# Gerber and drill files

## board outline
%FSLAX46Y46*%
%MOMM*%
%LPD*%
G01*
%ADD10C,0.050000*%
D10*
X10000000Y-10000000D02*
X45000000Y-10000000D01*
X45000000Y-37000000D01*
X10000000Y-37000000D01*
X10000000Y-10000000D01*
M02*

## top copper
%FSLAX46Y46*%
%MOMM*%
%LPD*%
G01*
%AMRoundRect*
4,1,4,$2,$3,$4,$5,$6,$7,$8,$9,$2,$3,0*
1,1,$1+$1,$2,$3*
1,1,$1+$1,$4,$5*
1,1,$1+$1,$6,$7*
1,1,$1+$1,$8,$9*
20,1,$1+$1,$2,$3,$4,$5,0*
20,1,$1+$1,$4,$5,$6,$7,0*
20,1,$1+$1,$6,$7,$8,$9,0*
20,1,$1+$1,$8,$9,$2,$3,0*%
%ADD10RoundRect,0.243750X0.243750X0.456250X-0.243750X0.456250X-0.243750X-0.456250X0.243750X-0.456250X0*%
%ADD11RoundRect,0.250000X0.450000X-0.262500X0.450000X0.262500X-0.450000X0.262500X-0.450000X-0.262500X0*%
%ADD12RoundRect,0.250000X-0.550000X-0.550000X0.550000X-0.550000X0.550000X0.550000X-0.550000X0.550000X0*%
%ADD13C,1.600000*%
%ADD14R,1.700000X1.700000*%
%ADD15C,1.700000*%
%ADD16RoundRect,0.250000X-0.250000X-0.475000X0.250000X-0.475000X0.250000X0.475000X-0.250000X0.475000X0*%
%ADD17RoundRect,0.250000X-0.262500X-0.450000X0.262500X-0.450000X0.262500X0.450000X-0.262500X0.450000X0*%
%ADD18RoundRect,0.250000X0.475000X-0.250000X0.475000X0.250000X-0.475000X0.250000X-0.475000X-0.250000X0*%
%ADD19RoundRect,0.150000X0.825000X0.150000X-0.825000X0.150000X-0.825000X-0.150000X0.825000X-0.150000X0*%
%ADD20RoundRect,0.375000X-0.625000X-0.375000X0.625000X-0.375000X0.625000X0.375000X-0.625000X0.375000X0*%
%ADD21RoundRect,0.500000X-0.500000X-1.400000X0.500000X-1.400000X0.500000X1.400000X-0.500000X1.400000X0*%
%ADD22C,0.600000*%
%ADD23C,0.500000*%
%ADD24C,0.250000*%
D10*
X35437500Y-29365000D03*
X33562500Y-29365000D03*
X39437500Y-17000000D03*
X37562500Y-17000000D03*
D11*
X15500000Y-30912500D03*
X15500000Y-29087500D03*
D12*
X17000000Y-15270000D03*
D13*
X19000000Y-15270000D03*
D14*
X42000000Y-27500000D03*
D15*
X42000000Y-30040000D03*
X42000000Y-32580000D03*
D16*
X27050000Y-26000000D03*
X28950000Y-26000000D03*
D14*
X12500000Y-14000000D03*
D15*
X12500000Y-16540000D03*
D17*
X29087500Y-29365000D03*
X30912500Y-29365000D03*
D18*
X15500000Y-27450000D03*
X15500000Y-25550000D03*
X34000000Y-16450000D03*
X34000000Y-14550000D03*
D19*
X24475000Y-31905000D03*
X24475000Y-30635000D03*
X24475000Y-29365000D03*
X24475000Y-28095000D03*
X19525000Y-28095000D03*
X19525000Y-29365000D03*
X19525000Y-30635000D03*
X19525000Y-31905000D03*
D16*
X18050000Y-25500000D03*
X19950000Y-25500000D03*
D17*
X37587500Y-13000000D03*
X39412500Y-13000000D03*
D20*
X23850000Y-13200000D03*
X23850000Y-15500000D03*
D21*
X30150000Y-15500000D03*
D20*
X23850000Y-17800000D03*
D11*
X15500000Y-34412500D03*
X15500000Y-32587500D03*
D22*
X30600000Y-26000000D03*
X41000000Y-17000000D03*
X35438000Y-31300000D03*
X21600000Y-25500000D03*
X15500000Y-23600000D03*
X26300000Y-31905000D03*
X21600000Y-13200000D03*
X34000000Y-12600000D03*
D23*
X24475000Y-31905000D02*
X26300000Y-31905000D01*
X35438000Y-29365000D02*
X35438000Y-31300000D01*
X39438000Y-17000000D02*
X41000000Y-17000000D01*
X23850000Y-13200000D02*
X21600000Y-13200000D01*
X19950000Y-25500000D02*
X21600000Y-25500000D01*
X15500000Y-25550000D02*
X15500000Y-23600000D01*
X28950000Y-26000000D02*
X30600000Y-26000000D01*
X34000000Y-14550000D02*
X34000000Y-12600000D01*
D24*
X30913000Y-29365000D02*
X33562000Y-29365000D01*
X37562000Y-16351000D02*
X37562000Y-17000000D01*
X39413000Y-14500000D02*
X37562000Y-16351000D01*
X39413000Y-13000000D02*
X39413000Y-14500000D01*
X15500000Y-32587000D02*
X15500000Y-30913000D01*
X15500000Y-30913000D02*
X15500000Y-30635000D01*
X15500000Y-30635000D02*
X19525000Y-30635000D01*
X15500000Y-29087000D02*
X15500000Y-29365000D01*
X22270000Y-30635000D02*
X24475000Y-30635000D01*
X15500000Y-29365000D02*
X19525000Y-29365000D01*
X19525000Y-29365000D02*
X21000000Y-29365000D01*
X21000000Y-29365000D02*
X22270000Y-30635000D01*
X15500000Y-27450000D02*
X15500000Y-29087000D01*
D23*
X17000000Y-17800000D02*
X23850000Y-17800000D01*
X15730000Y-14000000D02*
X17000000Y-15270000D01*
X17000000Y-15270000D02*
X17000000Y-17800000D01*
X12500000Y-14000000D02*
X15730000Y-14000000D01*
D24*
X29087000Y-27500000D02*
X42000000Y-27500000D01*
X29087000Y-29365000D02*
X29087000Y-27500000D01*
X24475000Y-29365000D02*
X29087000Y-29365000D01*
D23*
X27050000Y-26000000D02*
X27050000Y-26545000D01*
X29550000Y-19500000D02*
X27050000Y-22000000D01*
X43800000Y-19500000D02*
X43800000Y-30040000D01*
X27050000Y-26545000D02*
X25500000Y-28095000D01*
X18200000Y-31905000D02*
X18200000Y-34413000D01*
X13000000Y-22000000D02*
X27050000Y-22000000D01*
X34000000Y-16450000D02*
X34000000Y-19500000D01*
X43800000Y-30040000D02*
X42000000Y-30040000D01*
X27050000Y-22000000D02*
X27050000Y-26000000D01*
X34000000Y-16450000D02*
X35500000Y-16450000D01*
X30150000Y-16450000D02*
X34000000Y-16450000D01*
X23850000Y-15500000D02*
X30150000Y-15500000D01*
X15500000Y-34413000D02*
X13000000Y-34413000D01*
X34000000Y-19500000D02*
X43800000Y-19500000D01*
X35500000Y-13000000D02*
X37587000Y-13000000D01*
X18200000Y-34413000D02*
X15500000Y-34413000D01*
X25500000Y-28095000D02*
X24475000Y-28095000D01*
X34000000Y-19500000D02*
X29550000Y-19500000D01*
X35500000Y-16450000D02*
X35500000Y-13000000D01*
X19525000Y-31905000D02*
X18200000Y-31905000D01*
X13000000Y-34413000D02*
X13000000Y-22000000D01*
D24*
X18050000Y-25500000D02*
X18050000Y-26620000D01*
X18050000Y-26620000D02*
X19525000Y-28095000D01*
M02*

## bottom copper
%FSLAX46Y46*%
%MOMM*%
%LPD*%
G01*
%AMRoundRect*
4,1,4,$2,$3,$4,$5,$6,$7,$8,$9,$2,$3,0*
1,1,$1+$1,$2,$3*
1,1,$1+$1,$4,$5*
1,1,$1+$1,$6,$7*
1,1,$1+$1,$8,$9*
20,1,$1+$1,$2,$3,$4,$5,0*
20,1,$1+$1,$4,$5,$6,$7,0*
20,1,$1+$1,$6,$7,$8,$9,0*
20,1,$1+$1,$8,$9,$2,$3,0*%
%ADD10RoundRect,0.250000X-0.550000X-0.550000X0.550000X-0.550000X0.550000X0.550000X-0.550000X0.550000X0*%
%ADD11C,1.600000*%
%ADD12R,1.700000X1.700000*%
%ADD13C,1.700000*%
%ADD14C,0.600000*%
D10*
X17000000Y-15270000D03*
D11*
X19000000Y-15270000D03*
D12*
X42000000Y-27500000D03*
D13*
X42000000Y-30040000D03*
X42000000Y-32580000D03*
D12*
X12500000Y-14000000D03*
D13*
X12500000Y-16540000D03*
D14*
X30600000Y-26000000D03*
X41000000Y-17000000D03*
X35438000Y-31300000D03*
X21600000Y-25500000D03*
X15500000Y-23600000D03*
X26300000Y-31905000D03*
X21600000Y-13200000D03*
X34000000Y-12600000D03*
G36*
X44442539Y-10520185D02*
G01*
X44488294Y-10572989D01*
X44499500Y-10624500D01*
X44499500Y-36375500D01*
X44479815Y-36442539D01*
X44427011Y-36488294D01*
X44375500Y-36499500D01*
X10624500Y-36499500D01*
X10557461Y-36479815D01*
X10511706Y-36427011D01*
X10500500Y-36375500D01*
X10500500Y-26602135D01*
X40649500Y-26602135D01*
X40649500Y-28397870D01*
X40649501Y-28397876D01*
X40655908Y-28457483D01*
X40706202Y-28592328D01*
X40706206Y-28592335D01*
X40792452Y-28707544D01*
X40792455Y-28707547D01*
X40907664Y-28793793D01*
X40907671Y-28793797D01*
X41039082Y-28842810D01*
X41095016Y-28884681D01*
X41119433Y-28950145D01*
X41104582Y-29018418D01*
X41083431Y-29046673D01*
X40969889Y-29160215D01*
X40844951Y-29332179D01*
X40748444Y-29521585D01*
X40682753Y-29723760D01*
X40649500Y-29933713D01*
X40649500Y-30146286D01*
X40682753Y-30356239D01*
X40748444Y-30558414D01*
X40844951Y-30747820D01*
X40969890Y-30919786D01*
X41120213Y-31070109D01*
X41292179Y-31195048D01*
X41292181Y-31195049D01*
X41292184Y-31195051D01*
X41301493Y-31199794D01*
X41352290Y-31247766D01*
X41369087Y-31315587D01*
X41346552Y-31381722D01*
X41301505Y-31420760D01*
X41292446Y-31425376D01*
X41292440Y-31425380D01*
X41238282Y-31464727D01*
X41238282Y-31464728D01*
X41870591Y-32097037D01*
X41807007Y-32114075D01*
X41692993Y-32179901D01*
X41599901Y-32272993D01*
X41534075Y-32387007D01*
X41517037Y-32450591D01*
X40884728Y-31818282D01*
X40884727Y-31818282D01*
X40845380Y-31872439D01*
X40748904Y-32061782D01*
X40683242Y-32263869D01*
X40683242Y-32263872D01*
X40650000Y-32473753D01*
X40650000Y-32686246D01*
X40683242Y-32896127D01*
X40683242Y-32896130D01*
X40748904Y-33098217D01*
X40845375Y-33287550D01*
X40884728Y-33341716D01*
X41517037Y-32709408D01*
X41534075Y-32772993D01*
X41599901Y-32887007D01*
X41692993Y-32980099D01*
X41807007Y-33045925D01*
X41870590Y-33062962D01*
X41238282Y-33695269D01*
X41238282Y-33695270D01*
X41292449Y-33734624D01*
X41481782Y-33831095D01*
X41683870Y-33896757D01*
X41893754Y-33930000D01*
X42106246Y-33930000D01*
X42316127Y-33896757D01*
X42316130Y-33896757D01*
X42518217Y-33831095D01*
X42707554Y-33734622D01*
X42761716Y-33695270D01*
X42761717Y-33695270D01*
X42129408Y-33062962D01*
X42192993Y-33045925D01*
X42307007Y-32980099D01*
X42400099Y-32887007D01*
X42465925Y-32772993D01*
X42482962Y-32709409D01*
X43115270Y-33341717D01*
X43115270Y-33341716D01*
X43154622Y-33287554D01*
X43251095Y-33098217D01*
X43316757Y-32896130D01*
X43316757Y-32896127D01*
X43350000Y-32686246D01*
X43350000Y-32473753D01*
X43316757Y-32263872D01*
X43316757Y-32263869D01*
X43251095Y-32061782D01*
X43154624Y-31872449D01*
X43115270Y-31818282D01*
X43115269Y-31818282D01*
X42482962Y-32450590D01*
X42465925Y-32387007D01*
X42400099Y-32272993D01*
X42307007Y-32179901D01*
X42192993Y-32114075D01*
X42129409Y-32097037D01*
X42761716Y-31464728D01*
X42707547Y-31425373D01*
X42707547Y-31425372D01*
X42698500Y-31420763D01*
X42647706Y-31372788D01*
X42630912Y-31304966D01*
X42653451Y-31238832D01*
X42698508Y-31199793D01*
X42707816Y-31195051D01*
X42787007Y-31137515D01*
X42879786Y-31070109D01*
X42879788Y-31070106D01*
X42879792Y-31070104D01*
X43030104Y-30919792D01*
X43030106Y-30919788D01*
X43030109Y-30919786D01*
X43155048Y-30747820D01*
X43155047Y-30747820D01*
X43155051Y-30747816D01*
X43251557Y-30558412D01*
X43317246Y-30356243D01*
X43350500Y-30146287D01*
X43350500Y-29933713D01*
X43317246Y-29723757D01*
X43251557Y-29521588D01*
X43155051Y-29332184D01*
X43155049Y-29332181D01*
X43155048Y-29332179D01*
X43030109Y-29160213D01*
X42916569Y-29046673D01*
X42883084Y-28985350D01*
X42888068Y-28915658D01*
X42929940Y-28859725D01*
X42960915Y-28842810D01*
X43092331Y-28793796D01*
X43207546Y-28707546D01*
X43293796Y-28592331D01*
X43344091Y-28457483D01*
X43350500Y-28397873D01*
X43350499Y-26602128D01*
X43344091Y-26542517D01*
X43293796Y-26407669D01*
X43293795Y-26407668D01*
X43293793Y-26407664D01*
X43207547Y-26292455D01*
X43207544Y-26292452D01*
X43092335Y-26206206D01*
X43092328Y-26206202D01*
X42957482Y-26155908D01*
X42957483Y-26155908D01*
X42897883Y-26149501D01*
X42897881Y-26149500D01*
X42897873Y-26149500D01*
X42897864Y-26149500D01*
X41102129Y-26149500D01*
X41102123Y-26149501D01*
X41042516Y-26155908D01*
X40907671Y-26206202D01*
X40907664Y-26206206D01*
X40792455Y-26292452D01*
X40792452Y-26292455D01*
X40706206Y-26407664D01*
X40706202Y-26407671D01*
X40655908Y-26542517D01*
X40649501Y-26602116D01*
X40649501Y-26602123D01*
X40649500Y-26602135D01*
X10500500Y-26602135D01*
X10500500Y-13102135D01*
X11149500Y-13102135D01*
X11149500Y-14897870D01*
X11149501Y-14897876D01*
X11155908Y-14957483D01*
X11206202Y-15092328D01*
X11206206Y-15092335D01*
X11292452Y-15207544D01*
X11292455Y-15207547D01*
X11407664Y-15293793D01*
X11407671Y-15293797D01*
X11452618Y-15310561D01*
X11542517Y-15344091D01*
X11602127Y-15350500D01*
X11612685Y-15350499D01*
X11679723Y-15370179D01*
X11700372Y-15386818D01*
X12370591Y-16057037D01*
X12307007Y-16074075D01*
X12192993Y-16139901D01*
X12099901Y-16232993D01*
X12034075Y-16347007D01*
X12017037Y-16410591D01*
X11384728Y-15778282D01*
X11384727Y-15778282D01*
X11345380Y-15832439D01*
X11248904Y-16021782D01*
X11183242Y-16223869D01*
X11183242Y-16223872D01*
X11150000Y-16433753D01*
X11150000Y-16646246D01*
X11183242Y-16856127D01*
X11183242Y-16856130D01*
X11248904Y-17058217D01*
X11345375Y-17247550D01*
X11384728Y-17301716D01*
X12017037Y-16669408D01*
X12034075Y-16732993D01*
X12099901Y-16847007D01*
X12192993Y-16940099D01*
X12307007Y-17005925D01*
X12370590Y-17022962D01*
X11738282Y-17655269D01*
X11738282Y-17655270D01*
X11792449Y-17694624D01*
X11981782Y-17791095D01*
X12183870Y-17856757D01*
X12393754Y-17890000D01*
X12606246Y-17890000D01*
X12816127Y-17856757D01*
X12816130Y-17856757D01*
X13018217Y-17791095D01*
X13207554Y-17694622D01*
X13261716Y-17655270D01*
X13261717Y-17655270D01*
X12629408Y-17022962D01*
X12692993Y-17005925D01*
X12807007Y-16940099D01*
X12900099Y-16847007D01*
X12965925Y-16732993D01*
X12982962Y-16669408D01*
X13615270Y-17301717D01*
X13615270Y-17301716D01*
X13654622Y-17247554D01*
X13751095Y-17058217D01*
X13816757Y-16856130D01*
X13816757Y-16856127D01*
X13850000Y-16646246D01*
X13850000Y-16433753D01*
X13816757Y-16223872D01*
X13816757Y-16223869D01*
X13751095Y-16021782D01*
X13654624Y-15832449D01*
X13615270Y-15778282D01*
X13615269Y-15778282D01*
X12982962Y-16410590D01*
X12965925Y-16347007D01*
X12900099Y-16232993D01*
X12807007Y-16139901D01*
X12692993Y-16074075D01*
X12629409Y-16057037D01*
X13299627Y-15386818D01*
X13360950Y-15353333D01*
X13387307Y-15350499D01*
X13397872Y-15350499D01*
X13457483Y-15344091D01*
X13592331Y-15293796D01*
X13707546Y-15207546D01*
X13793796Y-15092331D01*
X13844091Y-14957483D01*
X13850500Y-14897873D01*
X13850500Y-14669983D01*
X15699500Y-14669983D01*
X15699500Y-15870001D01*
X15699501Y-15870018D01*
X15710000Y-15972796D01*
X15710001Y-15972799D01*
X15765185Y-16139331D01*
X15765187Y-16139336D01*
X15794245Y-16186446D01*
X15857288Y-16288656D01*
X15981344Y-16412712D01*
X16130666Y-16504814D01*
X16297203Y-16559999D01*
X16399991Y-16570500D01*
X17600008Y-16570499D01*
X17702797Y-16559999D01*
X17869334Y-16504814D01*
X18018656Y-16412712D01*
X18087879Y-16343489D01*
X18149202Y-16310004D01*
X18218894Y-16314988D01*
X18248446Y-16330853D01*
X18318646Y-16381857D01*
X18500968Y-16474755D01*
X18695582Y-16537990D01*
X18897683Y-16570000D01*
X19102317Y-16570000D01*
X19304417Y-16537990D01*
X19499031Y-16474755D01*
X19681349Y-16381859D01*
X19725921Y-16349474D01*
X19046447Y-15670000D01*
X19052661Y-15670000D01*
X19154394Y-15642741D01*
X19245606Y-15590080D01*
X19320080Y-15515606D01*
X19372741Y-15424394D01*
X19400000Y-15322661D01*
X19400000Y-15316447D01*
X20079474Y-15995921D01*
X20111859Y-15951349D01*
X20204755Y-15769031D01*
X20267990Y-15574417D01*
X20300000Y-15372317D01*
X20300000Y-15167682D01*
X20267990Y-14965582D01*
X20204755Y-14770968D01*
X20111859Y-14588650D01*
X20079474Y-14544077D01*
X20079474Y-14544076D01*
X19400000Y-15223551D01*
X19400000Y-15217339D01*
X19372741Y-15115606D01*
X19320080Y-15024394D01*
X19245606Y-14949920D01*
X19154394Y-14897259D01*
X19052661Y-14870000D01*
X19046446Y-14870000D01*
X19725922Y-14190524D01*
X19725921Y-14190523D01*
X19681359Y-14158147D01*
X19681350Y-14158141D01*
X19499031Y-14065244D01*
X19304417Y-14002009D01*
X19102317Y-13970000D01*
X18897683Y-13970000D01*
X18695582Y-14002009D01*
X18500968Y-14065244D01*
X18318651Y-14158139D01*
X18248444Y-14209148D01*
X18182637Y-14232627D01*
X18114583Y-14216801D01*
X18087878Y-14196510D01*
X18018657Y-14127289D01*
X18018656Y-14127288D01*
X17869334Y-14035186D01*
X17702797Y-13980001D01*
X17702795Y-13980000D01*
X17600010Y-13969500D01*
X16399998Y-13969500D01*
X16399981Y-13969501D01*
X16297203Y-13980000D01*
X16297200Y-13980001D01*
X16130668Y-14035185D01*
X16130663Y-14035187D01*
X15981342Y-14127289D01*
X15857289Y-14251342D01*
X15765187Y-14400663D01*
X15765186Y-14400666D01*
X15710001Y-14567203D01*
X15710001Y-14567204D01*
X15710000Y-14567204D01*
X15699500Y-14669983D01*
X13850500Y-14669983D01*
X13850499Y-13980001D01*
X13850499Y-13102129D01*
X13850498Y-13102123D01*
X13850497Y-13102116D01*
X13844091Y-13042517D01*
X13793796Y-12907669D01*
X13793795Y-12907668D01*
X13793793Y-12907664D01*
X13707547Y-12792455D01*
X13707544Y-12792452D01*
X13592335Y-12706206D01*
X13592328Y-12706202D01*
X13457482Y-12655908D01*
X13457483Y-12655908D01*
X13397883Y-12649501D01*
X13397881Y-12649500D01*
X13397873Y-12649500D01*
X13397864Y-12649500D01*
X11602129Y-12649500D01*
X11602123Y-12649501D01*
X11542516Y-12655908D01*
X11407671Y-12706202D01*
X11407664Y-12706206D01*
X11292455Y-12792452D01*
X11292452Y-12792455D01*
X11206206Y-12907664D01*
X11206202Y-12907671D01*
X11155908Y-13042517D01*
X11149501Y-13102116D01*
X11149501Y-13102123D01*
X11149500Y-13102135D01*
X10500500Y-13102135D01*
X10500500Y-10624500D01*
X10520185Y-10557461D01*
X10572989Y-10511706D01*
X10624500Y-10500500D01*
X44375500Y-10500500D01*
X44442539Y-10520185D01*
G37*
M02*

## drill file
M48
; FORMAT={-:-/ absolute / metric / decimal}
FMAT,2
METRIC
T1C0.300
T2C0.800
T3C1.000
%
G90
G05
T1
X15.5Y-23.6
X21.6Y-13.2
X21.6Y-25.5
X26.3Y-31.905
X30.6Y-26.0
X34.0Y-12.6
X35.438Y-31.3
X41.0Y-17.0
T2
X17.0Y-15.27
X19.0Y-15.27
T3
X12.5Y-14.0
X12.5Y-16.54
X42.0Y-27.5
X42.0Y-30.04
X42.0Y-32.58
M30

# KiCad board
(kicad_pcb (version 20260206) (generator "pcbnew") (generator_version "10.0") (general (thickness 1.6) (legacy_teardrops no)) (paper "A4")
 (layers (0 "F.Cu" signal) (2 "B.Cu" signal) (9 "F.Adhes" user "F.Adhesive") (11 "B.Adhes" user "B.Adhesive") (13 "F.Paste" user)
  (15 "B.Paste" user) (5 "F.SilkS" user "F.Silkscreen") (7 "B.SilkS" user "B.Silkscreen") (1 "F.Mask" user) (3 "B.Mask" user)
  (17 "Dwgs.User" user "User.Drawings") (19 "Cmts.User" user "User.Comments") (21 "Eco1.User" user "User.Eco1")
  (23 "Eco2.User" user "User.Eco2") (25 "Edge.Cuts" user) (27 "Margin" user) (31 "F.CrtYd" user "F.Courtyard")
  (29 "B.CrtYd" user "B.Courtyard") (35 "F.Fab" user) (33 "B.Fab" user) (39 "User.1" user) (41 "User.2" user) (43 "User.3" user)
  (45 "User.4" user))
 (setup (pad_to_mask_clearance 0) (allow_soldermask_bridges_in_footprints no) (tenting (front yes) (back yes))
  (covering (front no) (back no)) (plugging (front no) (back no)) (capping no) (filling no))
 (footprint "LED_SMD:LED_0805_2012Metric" (layer "F.Cu") (at 34.5 29.365 180)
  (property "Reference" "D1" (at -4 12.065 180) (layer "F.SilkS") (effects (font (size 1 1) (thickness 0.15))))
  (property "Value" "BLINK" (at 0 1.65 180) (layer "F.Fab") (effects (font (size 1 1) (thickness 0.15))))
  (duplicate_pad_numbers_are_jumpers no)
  (pad "1" smd roundrect (at -0.9375 0 180) (size 0.975 1.4) (layers "F.Cu" "F.Mask" "F.Paste") (roundrect_rratio 0.25) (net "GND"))
  (pad "2" smd roundrect (at 0.9375 0 180) (size 0.975 1.4) (layers "F.Cu" "F.Mask" "F.Paste") (roundrect_rratio 0.25) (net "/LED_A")))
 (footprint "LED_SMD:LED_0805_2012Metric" (layer "F.Cu") (at 38.5 17 180)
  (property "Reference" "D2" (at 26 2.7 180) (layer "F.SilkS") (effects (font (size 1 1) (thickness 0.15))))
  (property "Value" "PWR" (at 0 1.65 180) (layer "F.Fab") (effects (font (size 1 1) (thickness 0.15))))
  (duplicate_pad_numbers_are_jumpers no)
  (pad "1" smd roundrect (at -0.9375 0 180) (size 0.975 1.4) (layers "F.Cu" "F.Mask" "F.Paste") (roundrect_rratio 0.25) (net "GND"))
  (pad "2" smd roundrect (at 0.9375 0 180) (size 0.975 1.4) (layers "F.Cu" "F.Mask" "F.Paste") (roundrect_rratio 0.25) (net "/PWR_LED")))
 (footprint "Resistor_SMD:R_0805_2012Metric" (layer "F.Cu") (at 15.5 30 90)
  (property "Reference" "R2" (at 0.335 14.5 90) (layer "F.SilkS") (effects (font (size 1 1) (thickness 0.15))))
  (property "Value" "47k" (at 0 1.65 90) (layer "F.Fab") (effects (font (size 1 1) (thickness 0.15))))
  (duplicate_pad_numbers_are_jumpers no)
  (pad "1" smd roundrect (at -0.9125 0 90) (size 1.025 1.4) (layers "F.Cu" "F.Mask" "F.Paste") (roundrect_rratio 0.243902) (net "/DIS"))
  (pad "2" smd roundrect (at 0.9125 0 90) (size 1.025 1.4) (layers "F.Cu" "F.Mask" "F.Paste") (roundrect_rratio 0.243902) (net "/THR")))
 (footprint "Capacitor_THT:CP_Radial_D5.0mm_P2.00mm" (layer "F.Cu") (at 17 15.27)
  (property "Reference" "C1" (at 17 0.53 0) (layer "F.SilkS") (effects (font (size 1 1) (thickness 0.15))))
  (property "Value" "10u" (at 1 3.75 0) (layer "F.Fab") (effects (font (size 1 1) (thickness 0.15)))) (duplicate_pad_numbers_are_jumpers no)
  (pad "1" thru_hole roundrect (at 0 0) (size 1.6 1.6) (drill 0.8) (layers "*.Cu" "*.Mask") (remove_unused_layers no)
   (roundrect_rratio 0.15625) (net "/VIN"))
  (pad "2" thru_hole circle (at 2 0) (size 1.6 1.6) (drill 0.8) (layers "*.Cu" "*.Mask") (remove_unused_layers no) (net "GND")))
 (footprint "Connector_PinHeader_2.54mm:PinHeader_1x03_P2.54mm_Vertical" (layer "F.Cu") (at 42 27.5)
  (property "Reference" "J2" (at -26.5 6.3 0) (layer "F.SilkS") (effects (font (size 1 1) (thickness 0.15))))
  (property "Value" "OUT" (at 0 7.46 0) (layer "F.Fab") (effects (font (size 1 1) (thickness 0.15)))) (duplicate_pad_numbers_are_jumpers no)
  (pad "1" thru_hole rect (at 0 0) (size 1.7 1.7) (drill 1) (layers "*.Cu" "*.Mask") (remove_unused_layers no) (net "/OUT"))
  (pad "2" thru_hole circle (at 0 2.54) (size 1.7 1.7) (drill 1) (layers "*.Cu" "*.Mask") (remove_unused_layers no) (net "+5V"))
  (pad "3" thru_hole circle (at 0 5.08) (size 1.7 1.7) (drill 1) (layers "*.Cu" "*.Mask") (remove_unused_layers no) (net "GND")))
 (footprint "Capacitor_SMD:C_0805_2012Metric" (layer "F.Cu") (at 28 26)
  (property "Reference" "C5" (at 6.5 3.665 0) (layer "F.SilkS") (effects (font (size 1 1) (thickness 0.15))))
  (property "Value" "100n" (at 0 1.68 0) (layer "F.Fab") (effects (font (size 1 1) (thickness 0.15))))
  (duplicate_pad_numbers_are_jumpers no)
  (pad "1" smd roundrect (at -0.95 0) (size 1 1.45) (layers "F.Cu" "F.Mask" "F.Paste") (roundrect_rratio 0.25) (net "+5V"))
  (pad "2" smd roundrect (at 0.95 0) (size 1 1.45) (layers "F.Cu" "F.Mask" "F.Paste") (roundrect_rratio 0.25) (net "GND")))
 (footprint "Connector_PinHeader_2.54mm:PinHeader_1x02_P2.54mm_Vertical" (layer "F.Cu") (at 12.5 14)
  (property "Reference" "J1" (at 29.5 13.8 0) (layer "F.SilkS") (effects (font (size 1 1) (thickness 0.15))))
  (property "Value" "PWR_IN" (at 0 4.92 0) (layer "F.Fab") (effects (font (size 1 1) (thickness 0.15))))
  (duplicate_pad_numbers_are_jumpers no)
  (pad "1" thru_hole rect (at 0 0) (size 1.7 1.7) (drill 1) (layers "*.Cu" "*.Mask") (remove_unused_layers no) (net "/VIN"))
  (pad "2" thru_hole circle (at 0 2.54) (size 1.7 1.7) (drill 1) (layers "*.Cu" "*.Mask") (remove_unused_layers no) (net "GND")))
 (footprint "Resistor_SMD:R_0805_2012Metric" (layer "F.Cu") (at 30 29.365)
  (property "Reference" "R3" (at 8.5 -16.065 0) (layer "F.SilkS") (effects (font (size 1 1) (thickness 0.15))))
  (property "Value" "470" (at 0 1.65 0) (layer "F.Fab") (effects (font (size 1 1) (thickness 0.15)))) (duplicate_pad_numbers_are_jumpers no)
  (pad "1" smd roundrect (at -0.9125 0) (size 1.025 1.4) (layers "F.Cu" "F.Mask" "F.Paste") (roundrect_rratio 0.243902) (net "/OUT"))
  (pad "2" smd roundrect (at 0.9125 0) (size 1.025 1.4) (layers "F.Cu" "F.Mask" "F.Paste") (roundrect_rratio 0.243902) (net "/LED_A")))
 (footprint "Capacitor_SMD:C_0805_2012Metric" (layer "F.Cu") (at 15.5 26.5 90)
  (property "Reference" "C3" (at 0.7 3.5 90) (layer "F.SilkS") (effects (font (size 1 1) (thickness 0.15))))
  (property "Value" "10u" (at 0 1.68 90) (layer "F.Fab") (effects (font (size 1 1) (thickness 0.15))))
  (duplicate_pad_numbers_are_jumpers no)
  (pad "1" smd roundrect (at -0.95 0 90) (size 1 1.45) (layers "F.Cu" "F.Mask" "F.Paste") (roundrect_rratio 0.25) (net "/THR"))
  (pad "2" smd roundrect (at 0.95 0 90) (size 1 1.45) (layers "F.Cu" "F.Mask" "F.Paste") (roundrect_rratio 0.25) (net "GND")))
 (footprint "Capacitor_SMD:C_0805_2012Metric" (layer "F.Cu") (at 34 15.5 90)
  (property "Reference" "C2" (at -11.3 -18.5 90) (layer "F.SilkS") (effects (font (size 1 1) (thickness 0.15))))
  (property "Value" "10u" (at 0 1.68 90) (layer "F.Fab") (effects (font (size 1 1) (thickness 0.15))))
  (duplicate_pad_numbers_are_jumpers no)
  (pad "1" smd roundrect (at -0.95 0 90) (size 1 1.45) (layers "F.Cu" "F.Mask" "F.Paste") (roundrect_rratio 0.25) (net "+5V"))
  (pad "2" smd roundrect (at 0.95 0 90) (size 1 1.45) (layers "F.Cu" "F.Mask" "F.Paste") (roundrect_rratio 0.25) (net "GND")))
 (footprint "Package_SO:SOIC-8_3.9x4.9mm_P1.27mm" (layer "F.Cu") (at 22 30 180)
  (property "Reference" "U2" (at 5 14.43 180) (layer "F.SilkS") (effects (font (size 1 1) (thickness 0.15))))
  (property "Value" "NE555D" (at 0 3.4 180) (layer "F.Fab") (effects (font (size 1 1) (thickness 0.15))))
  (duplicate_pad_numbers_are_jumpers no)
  (pad "1" smd roundrect (at -2.475 -1.905 180) (size 1.95 0.6) (layers "F.Cu" "F.Mask" "F.Paste") (roundrect_rratio 0.25) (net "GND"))
  (pad "2" smd roundrect (at -2.475 -0.635 180) (size 1.95 0.6) (layers "F.Cu" "F.Mask" "F.Paste") (roundrect_rratio 0.25) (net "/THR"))
  (pad "3" smd roundrect (at -2.475 0.635 180) (size 1.95 0.6) (layers "F.Cu" "F.Mask" "F.Paste") (roundrect_rratio 0.25) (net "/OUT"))
  (pad "4" smd roundrect (at -2.475 1.905 180) (size 1.95 0.6) (layers "F.Cu" "F.Mask" "F.Paste") (roundrect_rratio 0.25) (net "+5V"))
  (pad "5" smd roundrect (at 2.475 1.905 180) (size 1.95 0.6) (layers "F.Cu" "F.Mask" "F.Paste") (roundrect_rratio 0.25) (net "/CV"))
  (pad "6" smd roundrect (at 2.475 0.635 180) (size 1.95 0.6) (layers "F.Cu" "F.Mask" "F.Paste") (roundrect_rratio 0.25) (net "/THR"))
  (pad "7" smd roundrect (at 2.475 -0.635 180) (size 1.95 0.6) (layers "F.Cu" "F.Mask" "F.Paste") (roundrect_rratio 0.25) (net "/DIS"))
  (pad "8" smd roundrect (at 2.475 -1.905 180) (size 1.95 0.6) (layers "F.Cu" "F.Mask" "F.Paste") (roundrect_rratio 0.25) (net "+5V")))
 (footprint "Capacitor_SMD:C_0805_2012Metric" (layer "F.Cu") (at 19 25.5)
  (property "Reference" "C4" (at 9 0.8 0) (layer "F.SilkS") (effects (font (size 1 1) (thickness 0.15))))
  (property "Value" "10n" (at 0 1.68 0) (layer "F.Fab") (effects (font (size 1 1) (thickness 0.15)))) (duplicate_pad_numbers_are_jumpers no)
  (pad "1" smd roundrect (at -0.95 0) (size 1 1.45) (layers "F.Cu" "F.Mask" "F.Paste") (roundrect_rratio 0.25) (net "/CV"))
  (pad "2" smd roundrect (at 0.95 0) (size 1 1.45) (layers "F.Cu" "F.Mask" "F.Paste") (roundrect_rratio 0.25) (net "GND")))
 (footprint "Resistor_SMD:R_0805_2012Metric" (layer "F.Cu") (at 38.5 13)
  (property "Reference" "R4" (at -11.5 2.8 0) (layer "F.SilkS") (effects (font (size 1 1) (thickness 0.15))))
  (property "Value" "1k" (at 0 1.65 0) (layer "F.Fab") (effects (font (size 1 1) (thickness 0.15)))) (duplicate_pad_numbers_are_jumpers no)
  (pad "1" smd roundrect (at -0.9125 0) (size 1.025 1.4) (layers "F.Cu" "F.Mask" "F.Paste") (roundrect_rratio 0.243902) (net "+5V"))
  (pad "2" smd roundrect (at 0.9125 0) (size 1.025 1.4) (layers "F.Cu" "F.Mask" "F.Paste") (roundrect_rratio 0.243902) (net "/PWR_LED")))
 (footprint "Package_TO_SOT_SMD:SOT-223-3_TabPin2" (layer "F.Cu") (at 27 15.5)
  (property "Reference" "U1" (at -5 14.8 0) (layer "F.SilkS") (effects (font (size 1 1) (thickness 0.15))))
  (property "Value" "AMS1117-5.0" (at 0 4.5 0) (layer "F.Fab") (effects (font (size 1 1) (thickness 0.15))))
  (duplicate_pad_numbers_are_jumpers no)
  (pad "1" smd roundrect (at -3.15 -2.3) (size 2 1.5) (layers "F.Cu" "F.Mask" "F.Paste") (roundrect_rratio 0.25) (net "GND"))
  (pad "2" smd roundrect (at -3.15 0) (size 2 1.5) (layers "F.Cu" "F.Mask" "F.Paste") (roundrect_rratio 0.25) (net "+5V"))
  (pad "2" smd roundrect (at 3.15 0) (size 2 3.8) (layers "F.Cu" "F.Mask" "F.Paste") (roundrect_rratio 0.25) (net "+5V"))
  (pad "3" smd roundrect (at -3.15 2.3) (size 2 1.5) (layers "F.Cu" "F.Mask" "F.Paste") (roundrect_rratio 0.25) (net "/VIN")))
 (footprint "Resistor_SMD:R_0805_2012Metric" (layer "F.Cu") (at 15.5 33.5 90)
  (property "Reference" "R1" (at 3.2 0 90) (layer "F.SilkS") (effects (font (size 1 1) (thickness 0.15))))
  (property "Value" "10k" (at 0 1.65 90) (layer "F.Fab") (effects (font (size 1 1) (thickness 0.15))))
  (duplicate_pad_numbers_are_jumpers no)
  (pad "1" smd roundrect (at -0.9125 0 90) (size 1.025 1.4) (layers "F.Cu" "F.Mask" "F.Paste") (roundrect_rratio 0.243902) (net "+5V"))
  (pad "2" smd roundrect (at 0.9125 0 90) (size 1.025 1.4) (layers "F.Cu" "F.Mask" "F.Paste") (roundrect_rratio 0.243902) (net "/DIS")))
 (gr_rect (start 10 10) (end 45 37) (stroke (width 0.05) (type default)) (fill no) (layer "Edge.Cuts"))
 (segment (start 24.475 31.905) (end 26.3 31.905) (width 0.5) (layer "F.Cu") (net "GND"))
 (segment (start 35.438 29.365) (end 35.438 31.3) (width 0.5) (layer "F.Cu") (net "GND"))
 (segment (start 39.438 17) (end 41 17) (width 0.5) (layer "F.Cu") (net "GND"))
 (segment (start 23.85 13.2) (end 21.6 13.2) (width 0.5) (layer "F.Cu") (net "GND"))
 (segment (start 19.95 25.5) (end 21.6 25.5) (width 0.5) (layer "F.Cu") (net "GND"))
 (segment (start 15.5 25.55) (end 15.5 23.6) (width 0.5) (layer "F.Cu") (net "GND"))
 (segment (start 28.95 26) (end 30.6 26) (width 0.5) (layer "F.Cu") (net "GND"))
 (segment (start 34 14.55) (end 34 12.6) (width 0.5) (layer "F.Cu") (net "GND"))
 (via (at 30.6 26) (size 0.6) (drill 0.3) (layers "F.Cu" "B.Cu") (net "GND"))
 (via (at 41 17) (size 0.6) (drill 0.3) (layers "F.Cu" "B.Cu") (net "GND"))
 (via (at 35.438 31.3) (size 0.6) (drill 0.3) (layers "F.Cu" "B.Cu") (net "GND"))
 (via (at 21.6 25.5) (size 0.6) (drill 0.3) (layers "F.Cu" "B.Cu") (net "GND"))
 (via (at 15.5 23.6) (size 0.6) (drill 0.3) (layers "F.Cu" "B.Cu") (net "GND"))
 (via (at 26.3 31.905) (size 0.6) (drill 0.3) (layers "F.Cu" "B.Cu") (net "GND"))
 (via (at 21.6 13.2) (size 0.6) (drill 0.3) (layers "F.Cu" "B.Cu") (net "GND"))
 (via (at 34 12.6) (size 0.6) (drill 0.3) (layers "F.Cu" "B.Cu") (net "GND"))
 (segment (start 30.913 29.365) (end 33.562 29.365) (width 0.25) (layer "F.Cu") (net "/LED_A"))
 (segment (start 37.562 16.351) (end 37.562 17) (width 0.25) (layer "F.Cu") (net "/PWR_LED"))
 (segment (start 39.413 14.5) (end 37.562 16.351) (width 0.25) (layer "F.Cu") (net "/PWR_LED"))
 (segment (start 39.413 13) (end 39.413 14.5) (width 0.25) (layer "F.Cu") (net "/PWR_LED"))
 (segment (start 15.5 32.587) (end 15.5 30.913) (width 0.25) (layer "F.Cu") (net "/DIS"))
 (segment (start 15.5 30.913) (end 15.5 30.635) (width 0.25) (layer "F.Cu") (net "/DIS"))
 (segment (start 15.5 30.635) (end 19.525 30.635) (width 0.25) (layer "F.Cu") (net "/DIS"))
 (segment (start 15.5 29.087) (end 15.5 29.365) (width 0.25) (layer "F.Cu") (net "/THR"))
 (segment (start 22.27 30.635) (end 24.475 30.635) (width 0.25) (layer "F.Cu") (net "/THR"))
 (segment (start 15.5 29.365) (end 19.525 29.365) (width 0.25) (layer "F.Cu") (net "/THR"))
 (segment (start 19.525 29.365) (end 21 29.365) (width 0.25) (layer "F.Cu") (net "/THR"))
 (segment (start 21 29.365) (end 22.27 30.635) (width 0.25) (layer "F.Cu") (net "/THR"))
 (segment (start 15.5 27.45) (end 15.5 29.087) (width 0.25) (layer "F.Cu") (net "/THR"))
 (segment (start 17 17.8) (end 23.85 17.8) (width 0.5) (layer "F.Cu") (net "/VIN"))
 (segment (start 15.73 14) (end 17 15.27) (width 0.5) (layer "F.Cu") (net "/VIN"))
 (segment (start 17 15.27) (end 17 17.8) (width 0.5) (layer "F.Cu") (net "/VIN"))
 (segment (start 12.5 14) (end 15.73 14) (width 0.5) (layer "F.Cu") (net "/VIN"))
 (segment (start 29.087 27.5) (end 42 27.5) (width 0.25) (layer "F.Cu") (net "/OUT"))
 (segment (start 29.087 29.365) (end 29.087 27.5) (width 0.25) (layer "F.Cu") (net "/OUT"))
 (segment (start 24.475 29.365) (end 29.087 29.365) (width 0.25) (layer "F.Cu") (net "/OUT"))
 (segment (start 27.05 26) (end 27.05 26.545) (width 0.5) (layer "F.Cu") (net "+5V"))
 (segment (start 29.55 19.5) (end 27.05 22) (width 0.5) (layer "F.Cu") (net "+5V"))
 (segment (start 43.8 19.5) (end 43.8 30.04) (width 0.5) (layer "F.Cu") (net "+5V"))
 (segment (start 27.05 26.545) (end 25.5 28.095) (width 0.5) (layer "F.Cu") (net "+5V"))
 (segment (start 18.2 31.905) (end 18.2 34.413) (width 0.5) (layer "F.Cu") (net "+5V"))
 (segment (start 13 22) (end 27.05 22) (width 0.5) (layer "F.Cu") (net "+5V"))
 (segment (start 34 16.45) (end 34 19.5) (width 0.5) (layer "F.Cu") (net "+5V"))
 (segment (start 43.8 30.04) (end 42 30.04) (width 0.5) (layer "F.Cu") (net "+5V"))
 (segment (start 27.05 22) (end 27.05 26) (width 0.5) (layer "F.Cu") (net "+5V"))
 (segment (start 34 16.45) (end 35.5 16.45) (width 0.5) (layer "F.Cu") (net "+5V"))
 (segment (start 30.15 16.45) (end 34 16.45) (width 0.5) (layer "F.Cu") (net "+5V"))
 (segment (start 23.85 15.5) (end 30.15 15.5) (width 0.5) (layer "F.Cu") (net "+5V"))
 (segment (start 15.5 34.413) (end 13 34.413) (width 0.5) (layer "F.Cu") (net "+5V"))
 (segment (start 34 19.5) (end 43.8 19.5) (width 0.5) (layer "F.Cu") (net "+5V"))
 (segment (start 35.5 13) (end 37.587 13) (width 0.5) (layer "F.Cu") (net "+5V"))
 (segment (start 18.2 34.413) (end 15.5 34.413) (width 0.5) (layer "F.Cu") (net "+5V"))
 (segment (start 25.5 28.095) (end 24.475 28.095) (width 0.5) (layer "F.Cu") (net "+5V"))
 (segment (start 34 19.5) (end 29.55 19.5) (width 0.5) (layer "F.Cu") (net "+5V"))
 (segment (start 35.5 16.45) (end 35.5 13) (width 0.5) (layer "F.Cu") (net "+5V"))
 (segment (start 19.525 31.905) (end 18.2 31.905) (width 0.5) (layer "F.Cu") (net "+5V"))
 (segment (start 13 34.413) (end 13 22) (width 0.5) (layer "F.Cu") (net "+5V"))
 (segment (start 18.05 25.5) (end 18.05 26.62) (width 0.25) (layer "F.Cu") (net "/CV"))
 (segment (start 18.05 26.62) (end 19.525 28.095) (width 0.25) (layer "F.Cu") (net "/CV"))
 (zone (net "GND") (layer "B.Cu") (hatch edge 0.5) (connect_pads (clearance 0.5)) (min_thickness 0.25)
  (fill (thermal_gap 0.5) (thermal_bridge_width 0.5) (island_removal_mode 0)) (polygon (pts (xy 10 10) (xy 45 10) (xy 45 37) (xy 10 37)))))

